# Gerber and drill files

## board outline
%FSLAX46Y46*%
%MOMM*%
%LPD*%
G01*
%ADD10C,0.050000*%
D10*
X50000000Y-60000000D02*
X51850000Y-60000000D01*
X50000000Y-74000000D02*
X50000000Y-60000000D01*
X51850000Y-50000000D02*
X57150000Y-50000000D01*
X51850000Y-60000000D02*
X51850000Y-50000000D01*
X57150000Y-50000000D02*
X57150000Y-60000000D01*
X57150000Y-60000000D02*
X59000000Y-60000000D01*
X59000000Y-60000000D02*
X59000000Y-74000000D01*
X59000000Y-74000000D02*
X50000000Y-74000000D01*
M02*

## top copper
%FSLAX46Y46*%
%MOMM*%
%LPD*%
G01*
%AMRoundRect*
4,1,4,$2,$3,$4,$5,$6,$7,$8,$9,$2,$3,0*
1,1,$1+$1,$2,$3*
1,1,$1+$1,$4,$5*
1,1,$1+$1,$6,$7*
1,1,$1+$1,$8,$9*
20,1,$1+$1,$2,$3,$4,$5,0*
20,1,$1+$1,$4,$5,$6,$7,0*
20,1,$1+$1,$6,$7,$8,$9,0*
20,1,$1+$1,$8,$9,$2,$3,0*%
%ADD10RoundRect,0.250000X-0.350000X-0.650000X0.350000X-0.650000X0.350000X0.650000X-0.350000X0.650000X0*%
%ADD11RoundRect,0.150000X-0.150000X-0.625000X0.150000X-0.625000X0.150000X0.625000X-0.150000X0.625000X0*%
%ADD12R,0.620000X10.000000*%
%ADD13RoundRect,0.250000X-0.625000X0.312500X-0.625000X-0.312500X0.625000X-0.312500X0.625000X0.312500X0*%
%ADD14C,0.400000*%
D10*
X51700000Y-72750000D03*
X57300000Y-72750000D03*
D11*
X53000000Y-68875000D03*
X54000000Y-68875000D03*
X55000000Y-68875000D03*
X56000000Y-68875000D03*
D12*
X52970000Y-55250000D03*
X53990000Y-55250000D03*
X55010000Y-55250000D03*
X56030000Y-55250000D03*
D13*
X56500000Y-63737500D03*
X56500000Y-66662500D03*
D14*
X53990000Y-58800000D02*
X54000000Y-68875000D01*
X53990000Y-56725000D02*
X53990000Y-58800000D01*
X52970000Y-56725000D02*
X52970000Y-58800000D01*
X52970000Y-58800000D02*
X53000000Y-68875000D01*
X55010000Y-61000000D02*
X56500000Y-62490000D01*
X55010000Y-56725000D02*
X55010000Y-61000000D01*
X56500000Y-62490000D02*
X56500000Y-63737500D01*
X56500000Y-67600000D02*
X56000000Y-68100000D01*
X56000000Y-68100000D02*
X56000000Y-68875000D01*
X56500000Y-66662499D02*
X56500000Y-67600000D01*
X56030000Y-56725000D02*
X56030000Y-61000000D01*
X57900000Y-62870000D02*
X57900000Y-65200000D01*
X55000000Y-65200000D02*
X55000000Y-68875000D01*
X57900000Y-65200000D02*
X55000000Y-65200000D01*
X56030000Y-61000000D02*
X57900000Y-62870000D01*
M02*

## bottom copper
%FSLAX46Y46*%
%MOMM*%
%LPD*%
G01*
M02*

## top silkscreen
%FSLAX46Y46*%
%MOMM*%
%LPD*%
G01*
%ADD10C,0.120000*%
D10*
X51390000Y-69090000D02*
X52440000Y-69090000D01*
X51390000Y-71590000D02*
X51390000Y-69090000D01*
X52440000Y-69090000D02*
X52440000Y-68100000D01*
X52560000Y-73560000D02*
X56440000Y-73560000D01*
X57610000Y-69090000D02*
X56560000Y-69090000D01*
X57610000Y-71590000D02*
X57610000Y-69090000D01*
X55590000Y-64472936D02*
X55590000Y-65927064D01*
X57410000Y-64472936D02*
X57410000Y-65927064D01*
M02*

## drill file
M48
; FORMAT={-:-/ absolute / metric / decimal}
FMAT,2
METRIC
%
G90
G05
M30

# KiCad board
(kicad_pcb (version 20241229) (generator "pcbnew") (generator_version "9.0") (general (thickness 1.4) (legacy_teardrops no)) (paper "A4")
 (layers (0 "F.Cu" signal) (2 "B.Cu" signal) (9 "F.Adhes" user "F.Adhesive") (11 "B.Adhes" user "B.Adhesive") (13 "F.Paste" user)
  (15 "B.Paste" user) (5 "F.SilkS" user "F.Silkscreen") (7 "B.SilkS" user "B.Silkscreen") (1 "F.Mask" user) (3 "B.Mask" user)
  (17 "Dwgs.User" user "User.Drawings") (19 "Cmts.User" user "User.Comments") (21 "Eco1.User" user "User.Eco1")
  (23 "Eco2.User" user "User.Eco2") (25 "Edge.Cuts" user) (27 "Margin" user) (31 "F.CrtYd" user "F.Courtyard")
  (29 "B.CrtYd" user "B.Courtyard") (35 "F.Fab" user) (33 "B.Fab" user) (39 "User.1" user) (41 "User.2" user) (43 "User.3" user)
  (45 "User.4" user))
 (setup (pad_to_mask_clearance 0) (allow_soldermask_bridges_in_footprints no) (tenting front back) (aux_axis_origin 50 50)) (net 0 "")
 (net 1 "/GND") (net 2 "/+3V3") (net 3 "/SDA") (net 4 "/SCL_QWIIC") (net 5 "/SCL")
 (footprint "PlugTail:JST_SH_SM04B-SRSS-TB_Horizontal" (layer "F.Cu") (at 54.5 70.875)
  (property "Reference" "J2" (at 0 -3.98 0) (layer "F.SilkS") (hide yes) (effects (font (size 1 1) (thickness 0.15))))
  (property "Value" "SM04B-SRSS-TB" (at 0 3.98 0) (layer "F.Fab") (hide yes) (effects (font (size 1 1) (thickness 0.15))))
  (fp_line (start -3.11 -1.785) (end -2.06 -1.785) (stroke (width 0.12) (type solid)) (layer "F.SilkS"))
  (fp_line (start -3.11 0.715) (end -3.11 -1.785) (stroke (width 0.12) (type solid)) (layer "F.SilkS"))
  (fp_line (start -2.06 -1.785) (end -2.06 -2.775) (stroke (width 0.12) (type solid)) (layer "F.SilkS"))
  (fp_line (start -1.94 2.685) (end 1.94 2.685) (stroke (width 0.12) (type solid)) (layer "F.SilkS"))
  (fp_line (start 3.11 -1.785) (end 2.06 -1.785) (stroke (width 0.12) (type solid)) (layer "F.SilkS"))
  (fp_line (start 3.11 0.715) (end 3.11 -1.785) (stroke (width 0.12) (type solid)) (layer "F.SilkS"))
  (pad "" smd roundrect (at -2.8 1.875) (size 1.2 1.8) (layers "F.Cu" "F.Mask" "F.Paste") (roundrect_rratio 0.208333))
  (pad "" smd roundrect (at 2.8 1.875) (size 1.2 1.8) (layers "F.Cu" "F.Mask" "F.Paste") (roundrect_rratio 0.208333))
  (pad "1" smd roundrect (at -1.5 -2) (size 0.6 1.55) (layers "F.Cu" "F.Mask" "F.Paste") (roundrect_rratio 0.25) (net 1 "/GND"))
  (pad "2" smd roundrect (at -0.5 -2) (size 0.6 1.55) (layers "F.Cu" "F.Mask" "F.Paste") (roundrect_rratio 0.25) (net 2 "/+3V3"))
  (pad "3" smd roundrect (at 0.5 -2) (size 0.6 1.55) (layers "F.Cu" "F.Mask" "F.Paste") (roundrect_rratio 0.25) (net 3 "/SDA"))
  (pad "4" smd roundrect (at 1.5 -2) (size 0.6 1.55) (layers "F.Cu" "F.Mask" "F.Paste") (roundrect_rratio 0.25) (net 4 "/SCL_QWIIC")))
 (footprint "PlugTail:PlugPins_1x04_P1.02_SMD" (layer "F.Cu") (at 54.5 50)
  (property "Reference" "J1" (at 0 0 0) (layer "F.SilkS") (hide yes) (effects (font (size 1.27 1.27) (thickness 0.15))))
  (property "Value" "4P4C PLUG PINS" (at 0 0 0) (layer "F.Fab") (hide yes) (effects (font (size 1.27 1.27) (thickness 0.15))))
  (pad "1" smd rect (at -1.53 5.25) (size 0.62 10) (layers "F.Cu" "F.Mask") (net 1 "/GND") (thermal_bridge_angle 45))
  (pad "2" smd rect (at -0.51 5.25) (size 0.62 10) (layers "F.Cu" "F.Mask") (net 2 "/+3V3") (thermal_bridge_angle 45))
  (pad "3" smd rect (at 0.51 5.25) (size 0.62 10) (layers "F.Cu" "F.Mask") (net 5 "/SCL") (thermal_bridge_angle 45))
  (pad "4" smd rect (at 1.53 5.25) (size 0.62 10) (layers "F.Cu" "F.Mask") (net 3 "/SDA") (thermal_bridge_angle 45)))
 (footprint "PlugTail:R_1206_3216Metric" (layer "F.Cu") (at 56.5 65.2 -90)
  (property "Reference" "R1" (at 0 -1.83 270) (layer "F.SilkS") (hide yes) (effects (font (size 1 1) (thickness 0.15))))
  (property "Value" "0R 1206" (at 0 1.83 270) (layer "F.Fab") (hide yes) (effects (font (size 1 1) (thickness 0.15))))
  (fp_line (start -0.727064 0.91) (end 0.727064 0.91) (stroke (width 0.12) (type solid)) (layer "F.SilkS"))
  (fp_line (start -0.727064 -0.91) (end 0.727064 -0.91) (stroke (width 0.12) (type solid)) (layer "F.SilkS"))
  (pad "1" smd roundrect (at -1.4625 0 270) (size 1.125 1.75) (layers "F.Cu" "F.Mask" "F.Paste") (roundrect_rratio 0.222222) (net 5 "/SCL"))
  (pad "2" smd roundrect (at 1.4625 0 270) (size 1.125 1.75) (layers "F.Cu" "F.Mask" "F.Paste") (roundrect_rratio 0.222222)
   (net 4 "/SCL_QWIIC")))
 (gr_line (start 50 60) (end 51.85 60) (stroke (width 0.05) (type default)) (layer "Edge.Cuts"))
 (gr_line (start 50 74) (end 50 60) (stroke (width 0.05) (type default)) (layer "Edge.Cuts"))
 (gr_line (start 51.85 50) (end 57.15 50) (stroke (width 0.05) (type default)) (layer "Edge.Cuts"))
 (gr_line (start 51.85 60) (end 51.85 50) (stroke (width 0.05) (type default)) (layer "Edge.Cuts"))
 (gr_line (start 57.15 50) (end 57.15 60) (stroke (width 0.05) (type default)) (layer "Edge.Cuts"))
 (gr_line (start 57.15 60) (end 59 60) (stroke (width 0.05) (type default)) (layer "Edge.Cuts"))
 (gr_line (start 59 60) (end 59 74) (stroke (width 0.05) (type default)) (layer "Edge.Cuts"))
 (gr_line (start 59 74) (end 50 74) (stroke (width 0.05) (type default)) (layer "Edge.Cuts"))
 (segment (start 53.99 58.8) (end 54 68.875) (width 0.4) (layer "F.Cu") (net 2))
 (segment (start 53.99 56.725) (end 53.99 58.8) (width 0.4) (layer "F.Cu") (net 2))
 (segment (start 52.97 56.725) (end 52.97 58.8) (width 0.4) (layer "F.Cu") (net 1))
 (segment (start 52.97 58.8) (end 53 68.875) (width 0.4) (layer "F.Cu") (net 1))
 (segment (start 55.01 61) (end 56.5 62.49) (width 0.4) (layer "F.Cu") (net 5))
 (segment (start 55.01 56.725) (end 55.01 61) (width 0.4) (layer "F.Cu") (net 5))
 (segment (start 56.5 62.49) (end 56.5 63.7375) (width 0.4) (layer "F.Cu") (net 5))
 (segment (start 56.5 67.6) (end 56 68.1) (width 0.4) (layer "F.Cu") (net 4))
 (segment (start 56 68.1) (end 56 68.875) (width 0.4) (layer "F.Cu") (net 4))
 (segment (start 56.5 66.662499) (end 56.5 67.6) (width 0.4) (layer "F.Cu") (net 4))
 (segment (start 56.03 56.725) (end 56.03 61) (width 0.4) (layer "F.Cu") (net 3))
 (segment (start 57.9 62.87) (end 57.9 65.2) (width 0.4) (layer "F.Cu") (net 3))
 (segment (start 55 65.2) (end 55 68.875) (width 0.4) (layer "F.Cu") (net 3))
 (segment (start 57.9 65.2) (end 55 65.2) (width 0.4) (layer "F.Cu") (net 3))
 (segment (start 56.03 61) (end 57.9 62.87) (width 0.4) (layer "F.Cu") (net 3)))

